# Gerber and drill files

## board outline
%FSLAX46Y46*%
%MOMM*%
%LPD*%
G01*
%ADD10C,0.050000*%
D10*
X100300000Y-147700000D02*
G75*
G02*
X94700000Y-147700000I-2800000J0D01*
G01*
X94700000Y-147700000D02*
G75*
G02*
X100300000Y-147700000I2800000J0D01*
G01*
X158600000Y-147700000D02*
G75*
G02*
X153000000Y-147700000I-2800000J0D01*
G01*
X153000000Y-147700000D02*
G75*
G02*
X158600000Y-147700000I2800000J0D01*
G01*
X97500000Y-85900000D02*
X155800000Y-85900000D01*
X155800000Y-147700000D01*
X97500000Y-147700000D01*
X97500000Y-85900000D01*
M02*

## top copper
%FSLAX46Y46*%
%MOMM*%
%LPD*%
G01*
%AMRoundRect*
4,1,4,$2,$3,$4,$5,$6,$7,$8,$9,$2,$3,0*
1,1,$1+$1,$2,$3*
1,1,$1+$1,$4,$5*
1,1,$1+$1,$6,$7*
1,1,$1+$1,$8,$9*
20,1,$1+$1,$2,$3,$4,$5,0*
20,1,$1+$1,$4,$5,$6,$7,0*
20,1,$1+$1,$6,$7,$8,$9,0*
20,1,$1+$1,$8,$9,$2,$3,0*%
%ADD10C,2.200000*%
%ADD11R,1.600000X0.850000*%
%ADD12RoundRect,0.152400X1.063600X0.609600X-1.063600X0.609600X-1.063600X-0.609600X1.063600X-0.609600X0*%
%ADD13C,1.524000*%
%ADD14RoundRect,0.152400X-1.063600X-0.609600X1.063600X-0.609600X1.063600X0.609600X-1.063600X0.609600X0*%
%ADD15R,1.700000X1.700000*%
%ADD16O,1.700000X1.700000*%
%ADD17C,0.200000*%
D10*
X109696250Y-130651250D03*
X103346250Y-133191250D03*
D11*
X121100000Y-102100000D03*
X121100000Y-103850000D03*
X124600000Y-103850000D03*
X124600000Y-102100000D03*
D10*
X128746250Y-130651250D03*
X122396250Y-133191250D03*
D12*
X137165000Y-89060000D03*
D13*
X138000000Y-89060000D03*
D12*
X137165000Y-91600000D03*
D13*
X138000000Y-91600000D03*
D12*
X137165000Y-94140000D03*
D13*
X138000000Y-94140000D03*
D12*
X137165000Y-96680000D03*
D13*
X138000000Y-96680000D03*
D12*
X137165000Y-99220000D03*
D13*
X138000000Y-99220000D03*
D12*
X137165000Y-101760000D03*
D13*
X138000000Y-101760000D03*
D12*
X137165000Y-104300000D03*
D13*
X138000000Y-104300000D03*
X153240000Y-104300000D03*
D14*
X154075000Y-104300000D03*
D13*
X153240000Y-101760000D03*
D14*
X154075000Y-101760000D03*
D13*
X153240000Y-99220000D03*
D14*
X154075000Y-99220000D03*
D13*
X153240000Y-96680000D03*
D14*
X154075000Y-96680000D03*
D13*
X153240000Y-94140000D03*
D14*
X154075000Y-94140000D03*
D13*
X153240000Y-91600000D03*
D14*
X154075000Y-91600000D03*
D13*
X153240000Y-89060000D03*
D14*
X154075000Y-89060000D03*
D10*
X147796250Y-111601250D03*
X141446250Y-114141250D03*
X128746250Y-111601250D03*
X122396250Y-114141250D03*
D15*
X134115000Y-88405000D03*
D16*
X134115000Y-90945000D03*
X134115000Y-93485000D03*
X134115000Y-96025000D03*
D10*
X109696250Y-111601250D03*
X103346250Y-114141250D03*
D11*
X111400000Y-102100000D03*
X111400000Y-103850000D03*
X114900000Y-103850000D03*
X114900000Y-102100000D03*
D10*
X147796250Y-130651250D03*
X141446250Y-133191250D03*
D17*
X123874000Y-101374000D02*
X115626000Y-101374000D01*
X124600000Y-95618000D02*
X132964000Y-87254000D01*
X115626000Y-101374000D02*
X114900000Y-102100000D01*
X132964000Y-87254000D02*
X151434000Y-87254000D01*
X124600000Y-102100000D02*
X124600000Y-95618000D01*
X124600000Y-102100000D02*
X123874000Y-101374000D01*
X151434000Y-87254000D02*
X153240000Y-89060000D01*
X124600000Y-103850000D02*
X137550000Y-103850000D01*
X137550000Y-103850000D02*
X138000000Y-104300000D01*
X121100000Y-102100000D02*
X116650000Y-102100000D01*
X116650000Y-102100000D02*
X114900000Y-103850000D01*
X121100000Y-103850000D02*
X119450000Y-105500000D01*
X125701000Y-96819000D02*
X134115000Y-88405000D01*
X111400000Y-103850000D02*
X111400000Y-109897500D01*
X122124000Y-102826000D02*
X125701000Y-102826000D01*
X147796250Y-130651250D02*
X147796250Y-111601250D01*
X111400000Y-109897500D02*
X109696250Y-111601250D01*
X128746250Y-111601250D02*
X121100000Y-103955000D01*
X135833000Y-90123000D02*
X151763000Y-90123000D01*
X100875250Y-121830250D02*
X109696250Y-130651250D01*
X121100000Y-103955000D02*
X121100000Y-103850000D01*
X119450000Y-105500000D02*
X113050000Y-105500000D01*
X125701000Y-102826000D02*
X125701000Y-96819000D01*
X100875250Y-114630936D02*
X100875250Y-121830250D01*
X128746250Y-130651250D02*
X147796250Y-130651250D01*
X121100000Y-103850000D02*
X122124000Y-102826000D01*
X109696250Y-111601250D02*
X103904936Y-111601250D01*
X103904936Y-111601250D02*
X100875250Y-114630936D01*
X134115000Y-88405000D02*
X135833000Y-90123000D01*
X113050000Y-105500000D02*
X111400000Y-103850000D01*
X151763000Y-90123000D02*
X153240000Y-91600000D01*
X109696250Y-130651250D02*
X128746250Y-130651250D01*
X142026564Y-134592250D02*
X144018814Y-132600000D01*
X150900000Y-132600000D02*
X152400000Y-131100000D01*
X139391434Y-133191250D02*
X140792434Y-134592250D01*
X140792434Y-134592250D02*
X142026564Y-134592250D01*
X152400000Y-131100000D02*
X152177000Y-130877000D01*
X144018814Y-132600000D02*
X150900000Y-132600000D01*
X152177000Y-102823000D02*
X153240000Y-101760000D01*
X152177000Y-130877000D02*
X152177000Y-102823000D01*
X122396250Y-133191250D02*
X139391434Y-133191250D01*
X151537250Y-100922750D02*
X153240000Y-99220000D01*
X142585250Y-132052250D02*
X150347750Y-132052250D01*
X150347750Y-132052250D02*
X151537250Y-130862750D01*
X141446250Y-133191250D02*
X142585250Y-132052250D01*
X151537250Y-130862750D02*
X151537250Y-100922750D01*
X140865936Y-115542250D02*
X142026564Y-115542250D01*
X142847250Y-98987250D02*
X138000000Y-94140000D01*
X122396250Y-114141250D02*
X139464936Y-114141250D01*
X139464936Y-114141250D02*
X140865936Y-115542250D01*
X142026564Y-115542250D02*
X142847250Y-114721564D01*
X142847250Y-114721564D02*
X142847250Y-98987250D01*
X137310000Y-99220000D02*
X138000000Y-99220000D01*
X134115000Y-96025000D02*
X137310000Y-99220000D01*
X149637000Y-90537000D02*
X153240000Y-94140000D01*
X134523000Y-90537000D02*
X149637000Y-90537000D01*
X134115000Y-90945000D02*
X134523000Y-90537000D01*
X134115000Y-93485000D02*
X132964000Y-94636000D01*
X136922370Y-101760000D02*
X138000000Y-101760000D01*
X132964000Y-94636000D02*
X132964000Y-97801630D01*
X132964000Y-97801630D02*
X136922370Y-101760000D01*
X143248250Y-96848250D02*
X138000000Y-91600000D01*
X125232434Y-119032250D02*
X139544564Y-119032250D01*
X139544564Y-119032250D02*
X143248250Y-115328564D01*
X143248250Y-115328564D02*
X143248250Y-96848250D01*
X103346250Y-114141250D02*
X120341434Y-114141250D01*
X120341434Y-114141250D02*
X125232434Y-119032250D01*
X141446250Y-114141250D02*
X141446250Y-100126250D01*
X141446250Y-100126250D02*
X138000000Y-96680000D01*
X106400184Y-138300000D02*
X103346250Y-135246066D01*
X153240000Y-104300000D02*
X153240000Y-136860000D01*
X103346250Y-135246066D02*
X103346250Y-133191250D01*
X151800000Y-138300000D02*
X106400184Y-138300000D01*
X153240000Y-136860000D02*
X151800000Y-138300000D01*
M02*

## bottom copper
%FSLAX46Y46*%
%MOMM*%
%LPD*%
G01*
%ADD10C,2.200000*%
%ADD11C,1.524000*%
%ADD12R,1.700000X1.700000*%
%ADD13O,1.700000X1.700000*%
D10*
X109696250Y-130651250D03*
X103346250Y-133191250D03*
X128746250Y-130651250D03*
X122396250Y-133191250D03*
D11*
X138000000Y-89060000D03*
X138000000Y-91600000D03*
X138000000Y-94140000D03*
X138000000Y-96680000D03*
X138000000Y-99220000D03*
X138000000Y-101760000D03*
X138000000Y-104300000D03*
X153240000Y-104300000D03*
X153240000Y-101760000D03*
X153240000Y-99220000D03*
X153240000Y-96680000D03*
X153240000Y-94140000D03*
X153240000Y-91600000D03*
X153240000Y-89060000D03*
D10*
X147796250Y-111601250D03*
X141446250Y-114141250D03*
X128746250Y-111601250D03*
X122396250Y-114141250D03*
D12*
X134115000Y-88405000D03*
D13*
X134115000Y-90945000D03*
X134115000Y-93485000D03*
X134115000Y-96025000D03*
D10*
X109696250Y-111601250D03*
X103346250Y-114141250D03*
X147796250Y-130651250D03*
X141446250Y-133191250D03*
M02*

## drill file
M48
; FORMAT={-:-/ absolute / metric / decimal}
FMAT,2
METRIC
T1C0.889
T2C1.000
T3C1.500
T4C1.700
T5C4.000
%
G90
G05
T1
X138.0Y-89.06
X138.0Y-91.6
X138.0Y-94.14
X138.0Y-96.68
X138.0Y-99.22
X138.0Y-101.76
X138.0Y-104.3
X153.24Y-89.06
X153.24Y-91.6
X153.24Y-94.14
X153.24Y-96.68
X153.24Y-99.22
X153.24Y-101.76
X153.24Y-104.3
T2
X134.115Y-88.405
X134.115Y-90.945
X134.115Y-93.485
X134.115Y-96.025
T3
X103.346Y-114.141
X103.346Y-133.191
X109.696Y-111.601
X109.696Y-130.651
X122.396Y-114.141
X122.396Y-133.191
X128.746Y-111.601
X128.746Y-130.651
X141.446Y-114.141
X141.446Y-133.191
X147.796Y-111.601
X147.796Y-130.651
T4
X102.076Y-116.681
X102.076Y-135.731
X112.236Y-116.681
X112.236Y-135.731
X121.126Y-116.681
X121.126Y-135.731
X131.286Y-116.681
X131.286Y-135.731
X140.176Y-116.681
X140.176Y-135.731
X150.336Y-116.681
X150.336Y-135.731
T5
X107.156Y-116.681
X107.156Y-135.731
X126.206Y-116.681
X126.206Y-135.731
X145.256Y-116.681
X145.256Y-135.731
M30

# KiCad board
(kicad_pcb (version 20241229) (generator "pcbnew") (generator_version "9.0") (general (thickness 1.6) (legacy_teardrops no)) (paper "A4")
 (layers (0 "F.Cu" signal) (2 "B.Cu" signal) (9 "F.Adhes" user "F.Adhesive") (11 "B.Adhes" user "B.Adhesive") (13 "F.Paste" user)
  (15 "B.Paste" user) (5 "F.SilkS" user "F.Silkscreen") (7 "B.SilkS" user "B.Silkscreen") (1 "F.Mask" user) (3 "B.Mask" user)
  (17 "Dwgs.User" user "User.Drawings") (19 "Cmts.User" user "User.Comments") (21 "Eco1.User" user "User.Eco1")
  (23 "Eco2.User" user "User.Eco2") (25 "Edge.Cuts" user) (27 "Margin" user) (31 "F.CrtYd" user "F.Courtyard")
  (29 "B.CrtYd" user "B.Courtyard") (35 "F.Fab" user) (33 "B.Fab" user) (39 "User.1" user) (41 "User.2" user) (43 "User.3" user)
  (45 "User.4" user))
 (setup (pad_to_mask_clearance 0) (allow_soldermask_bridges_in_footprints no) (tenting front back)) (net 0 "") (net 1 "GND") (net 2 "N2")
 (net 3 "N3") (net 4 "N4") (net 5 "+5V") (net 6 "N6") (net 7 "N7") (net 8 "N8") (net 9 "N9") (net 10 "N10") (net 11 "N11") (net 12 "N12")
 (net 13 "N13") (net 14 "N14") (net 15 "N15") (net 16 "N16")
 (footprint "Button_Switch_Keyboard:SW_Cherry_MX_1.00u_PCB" (layer "F.Cu") (at 109.69625 130.65125)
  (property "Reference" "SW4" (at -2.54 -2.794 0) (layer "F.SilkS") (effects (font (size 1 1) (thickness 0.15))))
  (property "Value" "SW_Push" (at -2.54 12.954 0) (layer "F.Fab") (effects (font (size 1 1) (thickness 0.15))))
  (pad "" np_thru_hole circle (at -7.62 5.08) (size 1.7 1.7) (drill 1.7) (layers "*.Cu" "*.Mask"))
  (pad "" np_thru_hole circle (at -2.54 5.08) (size 4 4) (drill 4) (layers "*.Cu" "*.Mask"))
  (pad "" np_thru_hole circle (at 2.54 5.08) (size 1.7 1.7) (drill 1.7) (layers "*.Cu" "*.Mask"))
  (pad "1" thru_hole circle (at 0 0) (size 2.2 2.2) (drill 1.5) (layers "*.Cu" "*.Mask") (remove_unused_layers no) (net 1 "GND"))
  (pad "2" thru_hole circle (at -6.35 2.54) (size 2.2 2.2) (drill 1.5) (layers "*.Cu" "*.Mask") (remove_unused_layers no) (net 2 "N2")))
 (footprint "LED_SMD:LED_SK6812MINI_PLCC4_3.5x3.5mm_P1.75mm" (layer "F.Cu") (at 122.85 102.975)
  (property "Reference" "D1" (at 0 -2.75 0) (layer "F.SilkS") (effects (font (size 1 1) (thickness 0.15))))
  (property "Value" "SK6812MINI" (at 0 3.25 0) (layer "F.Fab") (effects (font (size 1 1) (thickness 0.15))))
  (pad "1" smd rect (at -1.75 -0.875) (size 1.6 0.85) (layers "F.Cu" "F.Mask" "F.Paste") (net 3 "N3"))
  (pad "2" smd rect (at -1.75 0.875) (size 1.6 0.85) (layers "F.Cu" "F.Mask" "F.Paste") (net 1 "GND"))
  (pad "3" smd rect (at 1.75 0.875) (size 1.6 0.85) (layers "F.Cu" "F.Mask" "F.Paste") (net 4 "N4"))
  (pad "4" smd rect (at 1.75 -0.875) (size 1.6 0.85) (layers "F.Cu" "F.Mask" "F.Paste") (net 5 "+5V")))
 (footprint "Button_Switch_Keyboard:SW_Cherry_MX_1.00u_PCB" (layer "F.Cu") (at 128.74625 130.65125)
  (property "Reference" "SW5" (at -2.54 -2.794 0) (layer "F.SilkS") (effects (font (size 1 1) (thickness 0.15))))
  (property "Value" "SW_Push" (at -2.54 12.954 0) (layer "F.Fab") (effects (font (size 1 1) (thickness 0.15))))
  (pad "" np_thru_hole circle (at -7.62 5.08) (size 1.7 1.7) (drill 1.7) (layers "*.Cu" "*.Mask"))
  (pad "" np_thru_hole circle (at -2.54 5.08) (size 4 4) (drill 4) (layers "*.Cu" "*.Mask"))
  (pad "" np_thru_hole circle (at 2.54 5.08) (size 1.7 1.7) (drill 1.7) (layers "*.Cu" "*.Mask"))
  (pad "1" thru_hole circle (at 0 0) (size 2.2 2.2) (drill 1.5) (layers "*.Cu" "*.Mask") (remove_unused_layers no) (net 1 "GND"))
  (pad "2" thru_hole circle (at -6.35 2.54) (size 2.2 2.2) (drill 1.5) (layers "*.Cu" "*.Mask") (remove_unused_layers no) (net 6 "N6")))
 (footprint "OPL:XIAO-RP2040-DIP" (layer "F.Cu") (at 145.62 96.68)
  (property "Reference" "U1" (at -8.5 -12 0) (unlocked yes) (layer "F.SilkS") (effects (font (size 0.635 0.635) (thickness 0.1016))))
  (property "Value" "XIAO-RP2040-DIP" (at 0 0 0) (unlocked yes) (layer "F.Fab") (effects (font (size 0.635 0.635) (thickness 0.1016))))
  (pad "1" smd roundrect (at -8.455 -7.62 180) (size 2.432 1.524) (layers "F.Cu" "F.Mask") (roundrect_rratio 0.1) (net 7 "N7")
   (thermal_bridge_angle 45))
  (pad "1" thru_hole circle (at -7.62 -7.62 180) (size 1.524 1.524) (drill 0.889) (layers "*.Cu" "*.Mask") (remove_unused_layers no)
   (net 7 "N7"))
  (pad "2" smd roundrect (at -8.455 -5.08 180) (size 2.432 1.524) (layers "F.Cu" "F.Mask") (roundrect_rratio 0.1) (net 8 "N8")
   (thermal_bridge_angle 45))
  (pad "2" thru_hole circle (at -7.62 -5.08 180) (size 1.524 1.524) (drill 0.889) (layers "*.Cu" "*.Mask") (remove_unused_layers no)
   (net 8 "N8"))
  (pad "3" smd roundrect (at -8.455 -2.54 180) (size 2.432 1.524) (layers "F.Cu" "F.Mask") (roundrect_rratio 0.1) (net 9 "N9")
   (thermal_bridge_angle 45))
  (pad "3" thru_hole circle (at -7.62 -2.54 180) (size 1.524 1.524) (drill 0.889) (layers "*.Cu" "*.Mask") (remove_unused_layers no)
   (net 9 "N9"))
  (pad "4" smd roundrect (at -8.455 0 180) (size 2.432 1.524) (layers "F.Cu" "F.Mask") (roundrect_rratio 0.1) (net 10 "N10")
   (thermal_bridge_angle 45))
  (pad "4" thru_hole circle (at -7.62 0 180) (size 1.524 1.524) (drill 0.889) (layers "*.Cu" "*.Mask") (remove_unused_layers no)
   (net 10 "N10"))
  (pad "5" smd roundrect (at -8.455 2.54 180) (size 2.432 1.524) (layers "F.Cu" "F.Mask") (roundrect_rratio 0.1) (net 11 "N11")
   (thermal_bridge_angle 45))
  (pad "5" thru_hole circle (at -7.62 2.54 180) (size 1.524 1.524) (drill 0.889) (layers "*.Cu" "*.Mask") (remove_unused_layers no)
   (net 11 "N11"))
  (pad "6" smd roundrect (at -8.455 5.08 180) (size 2.432 1.524) (layers "F.Cu" "F.Mask") (roundrect_rratio 0.1) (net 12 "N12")
   (thermal_bridge_angle 45))
  (pad "6" thru_hole circle (at -7.62 5.08 180) (size 1.524 1.524) (drill 0.889) (layers "*.Cu" "*.Mask") (remove_unused_layers no)
   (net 12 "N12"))
  (pad "7" smd roundrect (at -8.455 7.62 180) (size 2.432 1.524) (layers "F.Cu" "F.Mask") (roundrect_rratio 0.1) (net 4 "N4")
   (thermal_bridge_angle 45))
  (pad "7" thru_hole circle (at -7.62 7.62 180) (size 1.524 1.524) (drill 0.889) (layers "*.Cu" "*.Mask") (remove_unused_layers no)
   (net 4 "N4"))
  (pad "8" thru_hole circle (at 7.62 7.62) (size 1.524 1.524) (drill 0.889) (layers "*.Cu" "*.Mask") (remove_unused_layers no) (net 2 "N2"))
  (pad "8" smd roundrect (at 8.455 7.62) (size 2.432 1.524) (layers "F.Cu" "F.Mask") (roundrect_rratio 0.1) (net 2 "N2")
   (thermal_bridge_angle 45))
  (pad "9" thru_hole circle (at 7.62 5.08) (size 1.524 1.524) (drill 0.889) (layers "*.Cu" "*.Mask") (remove_unused_layers no) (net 6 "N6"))
  (pad "9" smd roundrect (at 8.455 5.08) (size 2.432 1.524) (layers "F.Cu" "F.Mask") (roundrect_rratio 0.1) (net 6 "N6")
   (thermal_bridge_angle 45))
  (pad "10" thru_hole circle (at 7.62 2.54) (size 1.524 1.524) (drill 0.889) (layers "*.Cu" "*.Mask") (remove_unused_layers no)
   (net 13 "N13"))
  (pad "10" smd roundrect (at 8.455 2.54) (size 2.432 1.524) (layers "F.Cu" "F.Mask") (roundrect_rratio 0.1) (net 13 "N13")
   (thermal_bridge_angle 45))
  (pad "11" thru_hole circle (at 7.62 0) (size 1.524 1.524) (drill 0.889) (layers "*.Cu" "*.Mask") (remove_unused_layers no) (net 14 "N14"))
  (pad "11" smd roundrect (at 8.455 0) (size 2.432 1.524) (layers "F.Cu" "F.Mask") (roundrect_rratio 0.1) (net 14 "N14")
   (thermal_bridge_angle 45))
  (pad "12" thru_hole circle (at 7.62 -2.54) (size 1.524 1.524) (drill 0.889) (layers "*.Cu" "*.Mask") (remove_unused_layers no)
   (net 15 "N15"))
  (pad "12" smd roundrect (at 8.455 -2.54) (size 2.432 1.524) (layers "F.Cu" "F.Mask") (roundrect_rratio 0.1) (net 15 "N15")
   (thermal_bridge_angle 45))
  (pad "13" thru_hole circle (at 7.62 -5.08) (size 1.524 1.524) (drill 0.889) (layers "*.Cu" "*.Mask") (remove_unused_layers no)
   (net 1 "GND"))
  (pad "13" smd roundrect (at 8.455 -5.08) (size 2.432 1.524) (layers "F.Cu" "F.Mask") (roundrect_rratio 0.1) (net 1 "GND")
   (thermal_bridge_angle 45))
  (pad "14" thru_hole circle (at 7.62 -7.62) (size 1.524 1.524) (drill 0.889) (layers "*.Cu" "*.Mask") (remove_unused_layers no)
   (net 5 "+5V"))
  (pad "14" smd roundrect (at 8.455 -7.62) (size 2.432 1.524) (layers "F.Cu" "F.Mask") (roundrect_rratio 0.1) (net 5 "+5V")
   (thermal_bridge_angle 45)))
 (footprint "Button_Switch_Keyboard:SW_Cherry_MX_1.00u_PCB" (layer "F.Cu") (at 147.79625 111.60125)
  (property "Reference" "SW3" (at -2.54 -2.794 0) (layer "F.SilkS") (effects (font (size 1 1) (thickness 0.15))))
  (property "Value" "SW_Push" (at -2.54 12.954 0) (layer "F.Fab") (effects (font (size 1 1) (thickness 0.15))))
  (pad "" np_thru_hole circle (at -7.62 5.08) (size 1.7 1.7) (drill 1.7) (layers "*.Cu" "*.Mask"))
  (pad "" np_thru_hole circle (at -2.54 5.08) (size 4 4) (drill 4) (layers "*.Cu" "*.Mask"))
  (pad "" np_thru_hole circle (at 2.54 5.08) (size 1.7 1.7) (drill 1.7) (layers "*.Cu" "*.Mask"))
  (pad "1" thru_hole circle (at 0 0) (size 2.2 2.2) (drill 1.5) (layers "*.Cu" "*.Mask") (remove_unused_layers no) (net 1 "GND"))
  (pad "2" thru_hole circle (at -6.35 2.54) (size 2.2 2.2) (drill 1.5) (layers "*.Cu" "*.Mask") (remove_unused_layers no) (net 10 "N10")))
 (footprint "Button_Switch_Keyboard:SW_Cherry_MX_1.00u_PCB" (layer "F.Cu") (at 128.74625 111.60125)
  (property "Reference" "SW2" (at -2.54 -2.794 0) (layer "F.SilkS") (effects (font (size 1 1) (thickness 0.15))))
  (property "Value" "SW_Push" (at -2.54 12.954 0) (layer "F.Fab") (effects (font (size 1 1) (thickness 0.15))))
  (pad "" np_thru_hole circle (at -7.62 5.08) (size 1.7 1.7) (drill 1.7) (layers "*.Cu" "*.Mask"))
  (pad "" np_thru_hole circle (at -2.54 5.08) (size 4 4) (drill 4) (layers "*.Cu" "*.Mask"))
  (pad "" np_thru_hole circle (at 2.54 5.08) (size 1.7 1.7) (drill 1.7) (layers "*.Cu" "*.Mask"))
  (pad "1" thru_hole circle (at 0 0) (size 2.2 2.2) (drill 1.5) (layers "*.Cu" "*.Mask") (remove_unused_layers no) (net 1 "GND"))
  (pad "2" thru_hole circle (at -6.35 2.54) (size 2.2 2.2) (drill 1.5) (layers "*.Cu" "*.Mask") (remove_unused_layers no) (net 9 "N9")))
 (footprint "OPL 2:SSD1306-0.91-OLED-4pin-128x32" (layer "F.Cu") (at 97.615 86.215)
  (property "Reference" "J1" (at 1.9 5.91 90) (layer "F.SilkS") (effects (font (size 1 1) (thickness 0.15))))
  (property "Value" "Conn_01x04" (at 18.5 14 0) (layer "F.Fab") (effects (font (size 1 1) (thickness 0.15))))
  (pad "1" thru_hole rect (at 36.5 2.19) (size 1.7 1.7) (drill 1) (layers "*.Cu" "*.Mask") (remove_unused_layers no) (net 1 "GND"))
  (pad "2" thru_hole oval (at 36.5 4.73) (size 1.7 1.7) (drill 1) (layers "*.Cu" "*.Mask") (remove_unused_layers no) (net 15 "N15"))
  (pad "3" thru_hole oval (at 36.5 7.27) (size 1.7 1.7) (drill 1) (layers "*.Cu" "*.Mask") (remove_unused_layers no) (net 12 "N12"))
  (pad "4" thru_hole oval (at 36.5 9.81) (size 1.7 1.7) (drill 1) (layers "*.Cu" "*.Mask") (remove_unused_layers no) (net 11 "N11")))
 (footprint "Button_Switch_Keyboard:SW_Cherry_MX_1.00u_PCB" (layer "F.Cu") (at 109.69625 111.60125)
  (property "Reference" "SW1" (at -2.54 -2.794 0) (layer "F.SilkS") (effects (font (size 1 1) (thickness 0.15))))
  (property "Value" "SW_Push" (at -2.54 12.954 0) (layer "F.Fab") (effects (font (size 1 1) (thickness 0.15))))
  (pad "" np_thru_hole circle (at -7.62 5.08) (size 1.7 1.7) (drill 1.7) (layers "*.Cu" "*.Mask"))
  (pad "" np_thru_hole circle (at -2.54 5.08) (size 4 4) (drill 4) (layers "*.Cu" "*.Mask"))
  (pad "" np_thru_hole circle (at 2.54 5.08) (size 1.7 1.7) (drill 1.7) (layers "*.Cu" "*.Mask"))
  (pad "1" thru_hole circle (at 0 0) (size 2.2 2.2) (drill 1.5) (layers "*.Cu" "*.Mask") (remove_unused_layers no) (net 1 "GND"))
  (pad "2" thru_hole circle (at -6.35 2.54) (size 2.2 2.2) (drill 1.5) (layers "*.Cu" "*.Mask") (remove_unused_layers no) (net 8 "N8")))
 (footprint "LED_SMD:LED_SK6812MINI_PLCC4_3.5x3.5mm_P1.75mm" (layer "F.Cu") (at 113.15 102.975)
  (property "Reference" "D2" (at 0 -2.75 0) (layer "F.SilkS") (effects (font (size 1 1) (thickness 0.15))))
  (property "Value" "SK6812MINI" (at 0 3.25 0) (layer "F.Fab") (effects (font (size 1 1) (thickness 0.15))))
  (pad "1" smd rect (at -1.75 -0.875) (size 1.6 0.85) (layers "F.Cu" "F.Mask" "F.Paste") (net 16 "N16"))
  (pad "2" smd rect (at -1.75 0.875) (size 1.6 0.85) (layers "F.Cu" "F.Mask" "F.Paste") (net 1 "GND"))
  (pad "3" smd rect (at 1.75 0.875) (size 1.6 0.85) (layers "F.Cu" "F.Mask" "F.Paste") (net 3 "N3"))
  (pad "4" smd rect (at 1.75 -0.875) (size 1.6 0.85) (layers "F.Cu" "F.Mask" "F.Paste") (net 5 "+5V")))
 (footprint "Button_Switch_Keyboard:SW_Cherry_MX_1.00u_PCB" (layer "F.Cu") (at 147.79625 130.65125)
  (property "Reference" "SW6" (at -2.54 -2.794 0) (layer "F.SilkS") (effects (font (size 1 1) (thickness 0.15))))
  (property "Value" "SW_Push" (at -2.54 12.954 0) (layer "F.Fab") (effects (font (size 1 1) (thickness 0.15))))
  (pad "" np_thru_hole circle (at -7.62 5.08) (size 1.7 1.7) (drill 1.7) (layers "*.Cu" "*.Mask"))
  (pad "" np_thru_hole circle (at -2.54 5.08) (size 4 4) (drill 4) (layers "*.Cu" "*.Mask"))
  (pad "" np_thru_hole circle (at 2.54 5.08) (size 1.7 1.7) (drill 1.7) (layers "*.Cu" "*.Mask"))
  (pad "1" thru_hole circle (at 0 0) (size 2.2 2.2) (drill 1.5) (layers "*.Cu" "*.Mask") (remove_unused_layers no) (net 1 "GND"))
  (pad "2" thru_hole circle (at -6.35 2.54) (size 2.2 2.2) (drill 1.5) (layers "*.Cu" "*.Mask") (remove_unused_layers no) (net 13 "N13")))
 (gr_circle (center 97.5 147.7) (end 97.5 150.5) (stroke (width 0.05) (type default)) (fill no) (layer "Edge.Cuts"))
 (gr_circle (center 155.8 147.7) (end 155.8 150.5) (stroke (width 0.05) (type default)) (fill no) (layer "Edge.Cuts"))
 (gr_rect (start 97.5 85.9) (end 155.8 147.7) (stroke (width 0.05) (type default)) (fill no) (layer "Edge.Cuts"))
 (segment (start 123.874 101.374) (end 115.626 101.374) (width 0.2) (layer "F.Cu") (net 5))
 (segment (start 124.6 95.618) (end 132.964 87.254) (width 0.2) (layer "F.Cu") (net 5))
 (segment (start 115.626 101.374) (end 114.9 102.1) (width 0.2) (layer "F.Cu") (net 5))
 (segment (start 132.964 87.254) (end 151.434 87.254) (width 0.2) (layer "F.Cu") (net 5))
 (segment (start 124.6 102.1) (end 124.6 95.618) (width 0.2) (layer "F.Cu") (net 5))
 (segment (start 124.6 102.1) (end 123.874 101.374) (width 0.2) (layer "F.Cu") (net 5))
 (segment (start 151.434 87.254) (end 153.24 89.06) (width 0.2) (layer "F.Cu") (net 5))
 (segment (start 124.6 103.85) (end 137.55 103.85) (width 0.2) (layer "F.Cu") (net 4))
 (segment (start 137.55 103.85) (end 138 104.3) (width 0.2) (layer "F.Cu") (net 4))
 (segment (start 121.1 102.1) (end 116.65 102.1) (width 0.2) (layer "F.Cu") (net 3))
 (segment (start 116.65 102.1) (end 114.9 103.85) (width 0.2) (layer "F.Cu") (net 3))
 (segment (start 121.1 103.85) (end 119.45 105.5) (width 0.2) (layer "F.Cu") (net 1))
 (segment (start 125.701 96.819) (end 134.115 88.405) (width 0.2) (layer "F.Cu") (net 1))
 (segment (start 111.4 103.85) (end 111.4 109.8975) (width 0.2) (layer "F.Cu") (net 1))
 (segment (start 122.124 102.826) (end 125.701 102.826) (width 0.2) (layer "F.Cu") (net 1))
 (segment (start 147.79625 130.65125) (end 147.79625 111.60125) (width 0.2) (layer "F.Cu") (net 1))
 (segment (start 111.4 109.8975) (end 109.69625 111.60125) (width 0.2) (layer "F.Cu") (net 1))
 (segment (start 128.74625 111.60125) (end 121.1 103.955) (width 0.2) (layer "F.Cu") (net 1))
 (segment (start 135.833 90.123) (end 151.763 90.123) (width 0.2) (layer "F.Cu") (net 1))
 (segment (start 100.87525 121.83025) (end 109.69625 130.65125) (width 0.2) (layer "F.Cu") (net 1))
 (segment (start 121.1 103.955) (end 121.1 103.85) (width 0.2) (layer "F.Cu") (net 1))
 (segment (start 119.45 105.5) (end 113.05 105.5) (width 0.2) (layer "F.Cu") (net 1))
 (segment (start 125.701 102.826) (end 125.701 96.819) (width 0.2) (layer "F.Cu") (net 1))
 (segment (start 100.87525 114.630936) (end 100.87525 121.83025) (width 0.2) (layer "F.Cu") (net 1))
 (segment (start 128.74625 130.65125) (end 147.79625 130.65125) (width 0.2) (layer "F.Cu") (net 1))
 (segment (start 121.1 103.85) (end 122.124 102.826) (width 0.2) (layer "F.Cu") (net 1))
 (segment (start 109.69625 111.60125) (end 103.904936 111.60125) (width 0.2) (layer "F.Cu") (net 1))
 (segment (start 103.904936 111.60125) (end 100.87525 114.630936) (width 0.2) (layer "F.Cu") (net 1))
 (segment (start 134.115 88.405) (end 135.833 90.123) (width 0.2) (layer "F.Cu") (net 1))
 (segment (start 113.05 105.5) (end 111.4 103.85) (width 0.2) (layer "F.Cu") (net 1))
 (segment (start 151.763 90.123) (end 153.24 91.6) (width 0.2) (layer "F.Cu") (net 1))
 (segment (start 109.69625 130.65125) (end 128.74625 130.65125) (width 0.2) (layer "F.Cu") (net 1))
 (segment (start 142.026564 134.59225) (end 144.018814 132.6) (width 0.2) (layer "F.Cu") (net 6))
 (segment (start 150.9 132.6) (end 152.4 131.1) (width 0.2) (layer "F.Cu") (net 6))
 (segment (start 139.391434 133.19125) (end 140.792434 134.59225) (width 0.2) (layer "F.Cu") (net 6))
 (segment (start 140.792434 134.59225) (end 142.026564 134.59225) (width 0.2) (layer "F.Cu") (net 6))
 (segment (start 152.4 131.1) (end 152.177 130.877) (width 0.2) (layer "F.Cu") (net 6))
 (segment (start 144.018814 132.6) (end 150.9 132.6) (width 0.2) (layer "F.Cu") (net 6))
 (segment (start 152.177 102.823) (end 153.24 101.76) (width 0.2) (layer "F.Cu") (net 6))
 (segment (start 152.177 130.877) (end 152.177 102.823) (width 0.2) (layer "F.Cu") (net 6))
 (segment (start 122.39625 133.19125) (end 139.391434 133.19125) (width 0.2) (layer "F.Cu") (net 6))
 (segment (start 151.53725 100.92275) (end 153.24 99.22) (width 0.2) (layer "F.Cu") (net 13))
 (segment (start 142.58525 132.05225) (end 150.34775 132.05225) (width 0.2) (layer "F.Cu") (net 13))
 (segment (start 150.34775 132.05225) (end 151.53725 130.86275) (width 0.2) (layer "F.Cu") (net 13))
 (segment (start 141.44625 133.19125) (end 142.58525 132.05225) (width 0.2) (layer "F.Cu") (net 13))
 (segment (start 151.53725 130.86275) (end 151.53725 100.92275) (width 0.2) (layer "F.Cu") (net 13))
 (segment (start 140.865936 115.54225) (end 142.026564 115.54225) (width 0.2) (layer "F.Cu") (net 9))
 (segment (start 142.84725 98.98725) (end 138 94.14) (width 0.2) (layer "F.Cu") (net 9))
 (segment (start 122.39625 114.14125) (end 139.464936 114.14125) (width 0.2) (layer "F.Cu") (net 9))
 (segment (start 139.464936 114.14125) (end 140.865936 115.54225) (width 0.2) (layer "F.Cu") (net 9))
 (segment (start 142.026564 115.54225) (end 142.84725 114.721564) (width 0.2) (layer "F.Cu") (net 9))
 (segment (start 142.84725 114.721564) (end 142.84725 98.98725) (width 0.2) (layer "F.Cu") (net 9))
 (segment (start 137.31 99.22) (end 138 99.22) (width 0.2) (layer "F.Cu") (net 11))
 (segment (start 134.115 96.025) (end 137.31 99.22) (width 0.2) (layer "F.Cu") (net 11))
 (segment (start 149.637 90.537) (end 153.24 94.14) (width 0.2) (layer "F.Cu") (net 15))
 (segment (start 134.523 90.537) (end 149.637 90.537) (width 0.2) (layer "F.Cu") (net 15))
 (segment (start 134.115 90.945) (end 134.523 90.537) (width 0.2) (layer "F.Cu") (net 15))
 (segment (start 134.115 93.485) (end 132.964 94.636) (width 0.2) (layer "F.Cu") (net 12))
 (segment (start 136.92237 101.76) (end 138 101.76) (width 0.2) (layer "F.Cu") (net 12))
 (segment (start 132.964 94.636) (end 132.964 97.80163) (width 0.2) (layer "F.Cu") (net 12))
 (segment (start 132.964 97.80163) (end 136.92237 101.76) (width 0.2) (layer "F.Cu") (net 12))
 (segment (start 143.24825 96.84825) (end 138 91.6) (width 0.2) (layer "F.Cu") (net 8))
 (segment (start 125.232434 119.03225) (end 139.544564 119.03225) (width 0.2) (layer "F.Cu") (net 8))
 (segment (start 139.544564 119.03225) (end 143.24825 115.328564) (width 0.2) (layer "F.Cu") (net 8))
 (segment (start 143.24825 115.328564) (end 143.24825 96.84825) (width 0.2) (layer "F.Cu") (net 8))
 (segment (start 103.34625 114.14125) (end 120.341434 114.14125) (width 0.2) (layer "F.Cu") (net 8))
 (segment (start 120.341434 114.14125) (end 125.232434 119.03225) (width 0.2) (layer "F.Cu") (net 8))
 (segment (start 141.44625 114.14125) (end 141.44625 100.12625) (width 0.2) (layer "F.Cu") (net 10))
 (segment (start 141.44625 100.12625) (end 138 96.68) (width 0.2) (layer "F.Cu") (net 10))
 (segment (start 106.400184 138.3) (end 103.34625 135.246066) (width 0.2) (layer "F.Cu") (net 2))
 (segment (start 153.24 104.3) (end 153.24 136.86) (width 0.2) (layer "F.Cu") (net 2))
 (segment (start 103.34625 135.246066) (end 103.34625 133.19125) (width 0.2) (layer "F.Cu") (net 2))
 (segment (start 151.8 138.3) (end 106.400184 138.3) (width 0.2) (layer "F.Cu") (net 2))
 (segment (start 153.24 136.86) (end 151.8 138.3) (width 0.2) (layer "F.Cu") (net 2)))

